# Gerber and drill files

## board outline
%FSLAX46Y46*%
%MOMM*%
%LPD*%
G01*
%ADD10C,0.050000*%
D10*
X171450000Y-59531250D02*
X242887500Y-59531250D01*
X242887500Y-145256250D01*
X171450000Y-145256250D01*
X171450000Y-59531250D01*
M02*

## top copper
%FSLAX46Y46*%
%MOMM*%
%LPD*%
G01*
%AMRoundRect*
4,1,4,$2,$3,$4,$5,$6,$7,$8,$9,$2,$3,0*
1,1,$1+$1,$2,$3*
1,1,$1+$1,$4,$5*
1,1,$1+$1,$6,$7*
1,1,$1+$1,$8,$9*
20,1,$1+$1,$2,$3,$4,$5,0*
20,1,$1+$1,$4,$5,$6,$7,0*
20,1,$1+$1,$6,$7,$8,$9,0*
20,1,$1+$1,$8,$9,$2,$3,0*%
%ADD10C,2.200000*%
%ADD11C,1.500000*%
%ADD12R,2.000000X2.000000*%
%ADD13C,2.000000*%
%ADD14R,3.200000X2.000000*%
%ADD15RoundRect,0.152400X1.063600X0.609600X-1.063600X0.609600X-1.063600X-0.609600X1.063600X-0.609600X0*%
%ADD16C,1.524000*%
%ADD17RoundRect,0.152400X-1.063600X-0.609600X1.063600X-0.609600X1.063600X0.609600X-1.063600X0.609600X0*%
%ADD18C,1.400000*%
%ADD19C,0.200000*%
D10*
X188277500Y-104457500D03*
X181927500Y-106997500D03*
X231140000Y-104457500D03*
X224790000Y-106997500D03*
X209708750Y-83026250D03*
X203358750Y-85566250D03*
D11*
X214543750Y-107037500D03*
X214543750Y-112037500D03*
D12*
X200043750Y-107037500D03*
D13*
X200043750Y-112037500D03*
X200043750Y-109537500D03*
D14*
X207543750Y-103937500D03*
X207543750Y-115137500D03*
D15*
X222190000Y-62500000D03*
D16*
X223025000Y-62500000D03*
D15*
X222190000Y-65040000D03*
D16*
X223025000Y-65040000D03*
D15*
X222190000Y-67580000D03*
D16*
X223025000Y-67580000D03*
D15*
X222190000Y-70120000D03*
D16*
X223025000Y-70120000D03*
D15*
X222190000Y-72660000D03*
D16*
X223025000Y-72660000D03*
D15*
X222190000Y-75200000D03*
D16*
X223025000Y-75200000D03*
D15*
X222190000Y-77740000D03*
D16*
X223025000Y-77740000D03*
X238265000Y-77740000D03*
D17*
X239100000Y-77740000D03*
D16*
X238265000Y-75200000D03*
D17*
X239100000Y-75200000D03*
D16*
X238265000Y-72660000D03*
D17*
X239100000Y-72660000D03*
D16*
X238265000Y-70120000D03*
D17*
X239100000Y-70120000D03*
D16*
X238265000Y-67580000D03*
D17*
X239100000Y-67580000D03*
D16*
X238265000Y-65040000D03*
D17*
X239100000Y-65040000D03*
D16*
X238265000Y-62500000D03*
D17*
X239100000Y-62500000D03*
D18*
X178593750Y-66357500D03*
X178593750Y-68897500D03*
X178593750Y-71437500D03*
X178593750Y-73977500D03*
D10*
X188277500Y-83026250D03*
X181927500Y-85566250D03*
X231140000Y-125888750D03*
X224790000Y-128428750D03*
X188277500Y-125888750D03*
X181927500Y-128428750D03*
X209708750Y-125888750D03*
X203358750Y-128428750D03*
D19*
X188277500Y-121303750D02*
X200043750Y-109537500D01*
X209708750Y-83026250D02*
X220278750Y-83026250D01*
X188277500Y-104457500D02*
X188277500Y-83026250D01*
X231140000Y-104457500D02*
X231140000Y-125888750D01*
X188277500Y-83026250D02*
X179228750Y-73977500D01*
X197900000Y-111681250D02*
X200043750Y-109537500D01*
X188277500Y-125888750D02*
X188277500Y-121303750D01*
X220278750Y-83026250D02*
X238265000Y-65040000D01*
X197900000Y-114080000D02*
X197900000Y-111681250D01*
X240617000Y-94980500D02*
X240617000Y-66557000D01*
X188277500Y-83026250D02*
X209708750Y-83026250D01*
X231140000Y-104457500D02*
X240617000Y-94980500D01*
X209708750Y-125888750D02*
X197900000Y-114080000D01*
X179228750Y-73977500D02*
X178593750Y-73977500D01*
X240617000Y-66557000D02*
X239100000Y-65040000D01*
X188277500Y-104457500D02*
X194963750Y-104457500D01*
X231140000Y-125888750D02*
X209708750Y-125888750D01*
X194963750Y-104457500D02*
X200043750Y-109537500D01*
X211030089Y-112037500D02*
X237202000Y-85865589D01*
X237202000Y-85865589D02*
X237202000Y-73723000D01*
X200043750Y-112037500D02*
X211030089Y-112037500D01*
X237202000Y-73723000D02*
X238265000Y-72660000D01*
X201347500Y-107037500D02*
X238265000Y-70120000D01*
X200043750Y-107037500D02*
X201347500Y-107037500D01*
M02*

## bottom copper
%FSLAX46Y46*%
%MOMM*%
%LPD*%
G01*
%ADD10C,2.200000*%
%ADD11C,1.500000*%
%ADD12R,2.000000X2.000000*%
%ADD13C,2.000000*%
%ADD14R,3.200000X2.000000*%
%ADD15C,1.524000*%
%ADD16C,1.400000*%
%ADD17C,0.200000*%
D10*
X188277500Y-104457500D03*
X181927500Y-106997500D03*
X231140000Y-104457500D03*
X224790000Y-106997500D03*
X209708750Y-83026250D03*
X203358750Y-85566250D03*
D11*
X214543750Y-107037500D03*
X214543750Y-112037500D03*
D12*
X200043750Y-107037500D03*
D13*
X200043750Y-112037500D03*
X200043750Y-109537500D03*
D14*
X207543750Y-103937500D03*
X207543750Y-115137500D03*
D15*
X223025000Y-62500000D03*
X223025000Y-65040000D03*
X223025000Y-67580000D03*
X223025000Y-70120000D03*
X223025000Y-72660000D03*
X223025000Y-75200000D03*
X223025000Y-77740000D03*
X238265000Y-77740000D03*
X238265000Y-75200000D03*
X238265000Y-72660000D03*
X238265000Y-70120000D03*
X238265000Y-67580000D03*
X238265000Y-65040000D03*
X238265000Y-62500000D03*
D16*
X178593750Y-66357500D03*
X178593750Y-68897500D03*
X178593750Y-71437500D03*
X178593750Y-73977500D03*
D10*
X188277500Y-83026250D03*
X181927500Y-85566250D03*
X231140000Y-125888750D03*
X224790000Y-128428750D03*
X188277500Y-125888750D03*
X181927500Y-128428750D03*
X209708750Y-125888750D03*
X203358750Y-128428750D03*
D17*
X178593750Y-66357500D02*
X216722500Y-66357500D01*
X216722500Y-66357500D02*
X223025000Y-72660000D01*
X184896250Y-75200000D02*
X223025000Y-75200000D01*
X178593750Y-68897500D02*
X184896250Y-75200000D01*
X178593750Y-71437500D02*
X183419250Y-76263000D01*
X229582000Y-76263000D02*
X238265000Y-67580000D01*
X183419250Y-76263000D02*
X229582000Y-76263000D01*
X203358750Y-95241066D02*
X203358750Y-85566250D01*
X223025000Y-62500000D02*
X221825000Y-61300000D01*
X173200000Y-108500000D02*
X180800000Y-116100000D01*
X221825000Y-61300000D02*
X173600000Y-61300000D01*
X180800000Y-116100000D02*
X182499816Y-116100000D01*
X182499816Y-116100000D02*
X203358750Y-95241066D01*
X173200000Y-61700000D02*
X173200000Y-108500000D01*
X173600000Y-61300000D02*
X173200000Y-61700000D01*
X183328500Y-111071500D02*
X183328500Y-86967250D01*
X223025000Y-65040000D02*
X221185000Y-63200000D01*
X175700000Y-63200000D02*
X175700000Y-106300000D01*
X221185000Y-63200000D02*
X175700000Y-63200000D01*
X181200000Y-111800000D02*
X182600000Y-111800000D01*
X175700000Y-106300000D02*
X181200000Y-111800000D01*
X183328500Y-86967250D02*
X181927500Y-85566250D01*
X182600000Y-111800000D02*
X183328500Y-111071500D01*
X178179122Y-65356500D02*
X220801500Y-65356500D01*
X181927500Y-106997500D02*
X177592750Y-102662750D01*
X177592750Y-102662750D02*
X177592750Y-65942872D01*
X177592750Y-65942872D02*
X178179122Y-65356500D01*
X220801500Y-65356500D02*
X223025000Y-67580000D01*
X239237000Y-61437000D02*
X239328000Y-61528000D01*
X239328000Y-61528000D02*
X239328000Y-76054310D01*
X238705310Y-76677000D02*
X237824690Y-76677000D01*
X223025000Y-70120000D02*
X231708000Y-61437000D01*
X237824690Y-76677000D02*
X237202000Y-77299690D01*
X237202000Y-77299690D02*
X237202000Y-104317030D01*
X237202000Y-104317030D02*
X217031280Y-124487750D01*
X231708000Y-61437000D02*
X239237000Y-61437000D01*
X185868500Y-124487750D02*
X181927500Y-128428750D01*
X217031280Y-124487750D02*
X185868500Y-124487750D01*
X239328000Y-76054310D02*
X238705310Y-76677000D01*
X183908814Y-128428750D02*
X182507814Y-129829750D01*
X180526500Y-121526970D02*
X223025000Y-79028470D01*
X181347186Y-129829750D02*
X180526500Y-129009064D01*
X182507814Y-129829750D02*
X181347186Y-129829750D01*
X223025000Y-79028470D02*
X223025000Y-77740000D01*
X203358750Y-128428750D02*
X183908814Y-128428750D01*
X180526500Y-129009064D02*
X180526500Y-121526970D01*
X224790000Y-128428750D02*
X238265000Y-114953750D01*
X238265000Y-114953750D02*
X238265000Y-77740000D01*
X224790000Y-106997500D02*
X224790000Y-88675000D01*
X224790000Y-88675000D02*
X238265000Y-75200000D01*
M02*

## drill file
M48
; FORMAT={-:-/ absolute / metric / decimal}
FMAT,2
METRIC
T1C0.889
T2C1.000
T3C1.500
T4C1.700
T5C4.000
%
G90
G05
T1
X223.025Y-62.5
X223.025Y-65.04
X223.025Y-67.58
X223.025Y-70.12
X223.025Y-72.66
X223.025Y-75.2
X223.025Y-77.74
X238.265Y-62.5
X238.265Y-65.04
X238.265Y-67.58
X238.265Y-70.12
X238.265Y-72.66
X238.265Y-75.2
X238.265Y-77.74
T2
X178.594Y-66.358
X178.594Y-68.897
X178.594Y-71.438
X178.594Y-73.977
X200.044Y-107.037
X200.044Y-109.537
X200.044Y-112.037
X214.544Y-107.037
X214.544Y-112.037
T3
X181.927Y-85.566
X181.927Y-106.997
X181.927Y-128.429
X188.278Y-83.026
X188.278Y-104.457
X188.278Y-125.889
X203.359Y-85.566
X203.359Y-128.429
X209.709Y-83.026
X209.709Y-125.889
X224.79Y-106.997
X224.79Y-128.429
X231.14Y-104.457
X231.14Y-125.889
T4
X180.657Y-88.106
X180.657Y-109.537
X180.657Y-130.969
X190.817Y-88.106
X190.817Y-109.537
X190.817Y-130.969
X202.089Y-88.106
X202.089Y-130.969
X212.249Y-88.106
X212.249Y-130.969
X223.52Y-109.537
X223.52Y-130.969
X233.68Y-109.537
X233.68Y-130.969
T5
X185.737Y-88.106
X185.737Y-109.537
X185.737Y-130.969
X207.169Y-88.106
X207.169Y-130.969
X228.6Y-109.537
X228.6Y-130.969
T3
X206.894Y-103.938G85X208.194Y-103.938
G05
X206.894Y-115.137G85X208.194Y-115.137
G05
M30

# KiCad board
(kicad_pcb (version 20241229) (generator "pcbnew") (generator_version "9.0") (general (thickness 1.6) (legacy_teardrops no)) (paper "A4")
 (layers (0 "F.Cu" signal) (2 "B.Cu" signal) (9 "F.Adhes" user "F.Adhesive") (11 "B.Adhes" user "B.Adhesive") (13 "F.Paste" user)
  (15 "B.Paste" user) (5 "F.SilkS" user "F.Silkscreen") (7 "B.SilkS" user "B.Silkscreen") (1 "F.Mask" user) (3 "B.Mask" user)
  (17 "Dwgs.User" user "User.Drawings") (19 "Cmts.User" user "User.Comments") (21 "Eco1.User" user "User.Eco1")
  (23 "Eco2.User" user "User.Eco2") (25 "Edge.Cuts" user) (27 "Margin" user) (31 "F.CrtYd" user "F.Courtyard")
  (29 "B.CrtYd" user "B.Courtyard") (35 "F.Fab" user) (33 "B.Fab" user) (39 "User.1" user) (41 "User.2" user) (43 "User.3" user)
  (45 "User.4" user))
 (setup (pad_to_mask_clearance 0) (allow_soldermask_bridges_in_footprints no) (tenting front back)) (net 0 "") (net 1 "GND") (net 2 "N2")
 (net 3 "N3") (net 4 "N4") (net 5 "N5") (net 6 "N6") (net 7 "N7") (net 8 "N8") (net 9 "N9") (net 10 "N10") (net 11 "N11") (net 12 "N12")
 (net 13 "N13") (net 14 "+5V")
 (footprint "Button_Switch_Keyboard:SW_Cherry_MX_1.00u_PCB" (layer "F.Cu") (at 188.2775 104.4575)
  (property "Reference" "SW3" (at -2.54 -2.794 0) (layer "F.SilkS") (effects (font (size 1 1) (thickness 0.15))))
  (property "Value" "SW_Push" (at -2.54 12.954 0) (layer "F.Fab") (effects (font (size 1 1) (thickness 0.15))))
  (pad "" np_thru_hole circle (at -7.62 5.08) (size 1.7 1.7) (drill 1.7) (layers "*.Cu" "*.Mask"))
  (pad "" np_thru_hole circle (at -2.54 5.08) (size 4 4) (drill 4) (layers "*.Cu" "*.Mask"))
  (pad "" np_thru_hole circle (at 2.54 5.08) (size 1.7 1.7) (drill 1.7) (layers "*.Cu" "*.Mask"))
  (pad "1" thru_hole circle (at 0 0) (size 2.2 2.2) (drill 1.5) (layers "*.Cu" "*.Mask") (remove_unused_layers no) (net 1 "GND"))
  (pad "2" thru_hole circle (at -6.35 2.54) (size 2.2 2.2) (drill 1.5) (layers "*.Cu" "*.Mask") (remove_unused_layers no) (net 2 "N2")))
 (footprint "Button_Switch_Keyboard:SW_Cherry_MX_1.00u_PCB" (layer "F.Cu") (at 231.14 104.4575)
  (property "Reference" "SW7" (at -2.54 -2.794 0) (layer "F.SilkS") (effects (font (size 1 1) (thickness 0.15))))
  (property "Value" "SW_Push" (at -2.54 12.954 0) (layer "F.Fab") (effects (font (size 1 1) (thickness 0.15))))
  (pad "" np_thru_hole circle (at -7.62 5.08) (size 1.7 1.7) (drill 1.7) (layers "*.Cu" "*.Mask"))
  (pad "" np_thru_hole circle (at -2.54 5.08) (size 4 4) (drill 4) (layers "*.Cu" "*.Mask"))
  (pad "" np_thru_hole circle (at 2.54 5.08) (size 1.7 1.7) (drill 1.7) (layers "*.Cu" "*.Mask"))
  (pad "1" thru_hole circle (at 0 0) (size 2.2 2.2) (drill 1.5) (layers "*.Cu" "*.Mask") (remove_unused_layers no) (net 1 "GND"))
  (pad "2" thru_hole circle (at -6.35 2.54) (size 2.2 2.2) (drill 1.5) (layers "*.Cu" "*.Mask") (remove_unused_layers no) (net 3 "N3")))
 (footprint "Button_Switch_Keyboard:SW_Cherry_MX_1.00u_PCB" (layer "F.Cu") (at 209.70875 83.02625)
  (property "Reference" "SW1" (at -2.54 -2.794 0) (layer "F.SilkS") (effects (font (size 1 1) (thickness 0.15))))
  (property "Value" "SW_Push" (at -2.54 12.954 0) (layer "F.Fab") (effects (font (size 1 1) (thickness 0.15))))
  (pad "" np_thru_hole circle (at -7.62 5.08) (size 1.7 1.7) (drill 1.7) (layers "*.Cu" "*.Mask"))
  (pad "" np_thru_hole circle (at -2.54 5.08) (size 4 4) (drill 4) (layers "*.Cu" "*.Mask"))
  (pad "" np_thru_hole circle (at 2.54 5.08) (size 1.7 1.7) (drill 1.7) (layers "*.Cu" "*.Mask"))
  (pad "1" thru_hole circle (at 0 0) (size 2.2 2.2) (drill 1.5) (layers "*.Cu" "*.Mask") (remove_unused_layers no) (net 1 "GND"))
  (pad "2" thru_hole circle (at -6.35 2.54) (size 2.2 2.2) (drill 1.5) (layers "*.Cu" "*.Mask") (remove_unused_layers no) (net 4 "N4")))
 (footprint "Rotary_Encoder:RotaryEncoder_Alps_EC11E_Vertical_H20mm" (layer "F.Cu") (at 200.04375 107.0375)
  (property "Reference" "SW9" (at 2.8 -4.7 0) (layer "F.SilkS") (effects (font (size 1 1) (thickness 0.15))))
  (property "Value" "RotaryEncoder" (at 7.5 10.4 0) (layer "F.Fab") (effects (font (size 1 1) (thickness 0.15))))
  (pad "" thru_hole circle (at 14.5 0) (size 1.5 1.5) (drill 1) (layers "*.Cu" "*.Mask") (remove_unused_layers no))
  (pad "" thru_hole circle (at 14.5 5) (size 1.5 1.5) (drill 1) (layers "*.Cu" "*.Mask") (remove_unused_layers no))
  (pad "A" thru_hole rect (at 0 0) (size 2 2) (drill 1) (layers "*.Cu" "*.Mask") (remove_unused_layers no) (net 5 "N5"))
  (pad "B" thru_hole circle (at 0 5) (size 2 2) (drill 1) (layers "*.Cu" "*.Mask") (remove_unused_layers no) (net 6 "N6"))
  (pad "C" thru_hole circle (at 0 2.5) (size 2 2) (drill 1) (layers "*.Cu" "*.Mask") (remove_unused_layers no) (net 1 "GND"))
  (pad "MP" thru_hole rect (at 7.5 -3.1) (size 3.2 2) (drill oval 2.8 1.5) (layers "*.Cu" "*.Mask") (remove_unused_layers no))
  (pad "MP" thru_hole rect (at 7.5 8.1) (size 3.2 2) (drill oval 2.8 1.5) (layers "*.Cu" "*.Mask") (remove_unused_layers no)))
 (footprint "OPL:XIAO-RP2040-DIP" (layer "F.Cu") (at 230.645 70.12)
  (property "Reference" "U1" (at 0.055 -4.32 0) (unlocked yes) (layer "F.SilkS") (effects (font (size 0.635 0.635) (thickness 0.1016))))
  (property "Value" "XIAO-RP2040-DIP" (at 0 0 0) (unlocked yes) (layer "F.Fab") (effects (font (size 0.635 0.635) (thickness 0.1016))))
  (pad "1" smd roundrect (at -8.455 -7.62 180) (size 2.432 1.524) (layers "F.Cu" "F.Mask") (roundrect_rratio 0.1) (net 4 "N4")
   (thermal_bridge_angle 45))
  (pad "1" thru_hole circle (at -7.62 -7.62 180) (size 1.524 1.524) (drill 0.889) (layers "*.Cu" "*.Mask") (remove_unused_layers no)
   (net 4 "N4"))
  (pad "2" smd roundrect (at -8.455 -5.08 180) (size 2.432 1.524) (layers "F.Cu" "F.Mask") (roundrect_rratio 0.1) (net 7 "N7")
   (thermal_bridge_angle 45))
  (pad "2" thru_hole circle (at -7.62 -5.08 180) (size 1.524 1.524) (drill 0.889) (layers "*.Cu" "*.Mask") (remove_unused_layers no)
   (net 7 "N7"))
  (pad "3" smd roundrect (at -8.455 -2.54 180) (size 2.432 1.524) (layers "F.Cu" "F.Mask") (roundrect_rratio 0.1) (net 2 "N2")
   (thermal_bridge_angle 45))
  (pad "3" thru_hole circle (at -7.62 -2.54 180) (size 1.524 1.524) (drill 0.889) (layers "*.Cu" "*.Mask") (remove_unused_layers no)
   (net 2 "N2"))
  (pad "4" smd roundrect (at -8.455 0 180) (size 2.432 1.524) (layers "F.Cu" "F.Mask") (roundrect_rratio 0.1) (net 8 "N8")
   (thermal_bridge_angle 45))
  (pad "4" thru_hole circle (at -7.62 0 180) (size 1.524 1.524) (drill 0.889) (layers "*.Cu" "*.Mask") (remove_unused_layers no)
   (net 8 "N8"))
  (pad "5" smd roundrect (at -8.455 2.54 180) (size 2.432 1.524) (layers "F.Cu" "F.Mask") (roundrect_rratio 0.1) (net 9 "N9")
   (thermal_bridge_angle 45))
  (pad "5" thru_hole circle (at -7.62 2.54 180) (size 1.524 1.524) (drill 0.889) (layers "*.Cu" "*.Mask") (remove_unused_layers no)
   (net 9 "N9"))
  (pad "6" smd roundrect (at -8.455 5.08 180) (size 2.432 1.524) (layers "F.Cu" "F.Mask") (roundrect_rratio 0.1) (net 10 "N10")
   (thermal_bridge_angle 45))
  (pad "6" thru_hole circle (at -7.62 5.08 180) (size 1.524 1.524) (drill 0.889) (layers "*.Cu" "*.Mask") (remove_unused_layers no)
   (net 10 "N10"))
  (pad "7" smd roundrect (at -8.455 7.62 180) (size 2.432 1.524) (layers "F.Cu" "F.Mask") (roundrect_rratio 0.1) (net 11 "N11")
   (thermal_bridge_angle 45))
  (pad "7" thru_hole circle (at -7.62 7.62 180) (size 1.524 1.524) (drill 0.889) (layers "*.Cu" "*.Mask") (remove_unused_layers no)
   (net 11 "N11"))
  (pad "8" thru_hole circle (at 7.62 7.62) (size 1.524 1.524) (drill 0.889) (layers "*.Cu" "*.Mask") (remove_unused_layers no)
   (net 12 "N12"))
  (pad "8" smd roundrect (at 8.455 7.62) (size 2.432 1.524) (layers "F.Cu" "F.Mask") (roundrect_rratio 0.1) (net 12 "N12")
   (thermal_bridge_angle 45))
  (pad "9" thru_hole circle (at 7.62 5.08) (size 1.524 1.524) (drill 0.889) (layers "*.Cu" "*.Mask") (remove_unused_layers no) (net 3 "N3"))
  (pad "9" smd roundrect (at 8.455 5.08) (size 2.432 1.524) (layers "F.Cu" "F.Mask") (roundrect_rratio 0.1) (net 3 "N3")
   (thermal_bridge_angle 45))
  (pad "10" thru_hole circle (at 7.62 2.54) (size 1.524 1.524) (drill 0.889) (layers "*.Cu" "*.Mask") (remove_unused_layers no) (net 6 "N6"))
  (pad "10" smd roundrect (at 8.455 2.54) (size 2.432 1.524) (layers "F.Cu" "F.Mask") (roundrect_rratio 0.1) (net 6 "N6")
   (thermal_bridge_angle 45))
  (pad "11" thru_hole circle (at 7.62 0) (size 1.524 1.524) (drill 0.889) (layers "*.Cu" "*.Mask") (remove_unused_layers no) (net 5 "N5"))
  (pad "11" smd roundrect (at 8.455 0) (size 2.432 1.524) (layers "F.Cu" "F.Mask") (roundrect_rratio 0.1) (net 5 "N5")
   (thermal_bridge_angle 45))
  (pad "12" thru_hole circle (at 7.62 -2.54) (size 1.524 1.524) (drill 0.889) (layers "*.Cu" "*.Mask") (remove_unused_layers no)
   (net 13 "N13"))
  (pad "12" smd roundrect (at 8.455 -2.54) (size 2.432 1.524) (layers "F.Cu" "F.Mask") (roundrect_rratio 0.1) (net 13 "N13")
   (thermal_bridge_angle 45))
  (pad "13" thru_hole circle (at 7.62 -5.08) (size 1.524 1.524) (drill 0.889) (layers "*.Cu" "*.Mask") (remove_unused_layers no)
   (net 1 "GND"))
  (pad "13" smd roundrect (at 8.455 -5.08) (size 2.432 1.524) (layers "F.Cu" "F.Mask") (roundrect_rratio 0.1) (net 1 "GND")
   (thermal_bridge_angle 45))
  (pad "14" thru_hole circle (at 7.62 -7.62) (size 1.524 1.524) (drill 0.889) (layers "*.Cu" "*.Mask") (remove_unused_layers no)
   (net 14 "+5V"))
  (pad "14" smd roundrect (at 8.455 -7.62) (size 2.432 1.524) (layers "F.Cu" "F.Mask") (roundrect_rratio 0.1) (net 14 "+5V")
   (thermal_bridge_angle 45)))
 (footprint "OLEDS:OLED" (layer "F.Cu") (at 178.59375 70.1675 -90)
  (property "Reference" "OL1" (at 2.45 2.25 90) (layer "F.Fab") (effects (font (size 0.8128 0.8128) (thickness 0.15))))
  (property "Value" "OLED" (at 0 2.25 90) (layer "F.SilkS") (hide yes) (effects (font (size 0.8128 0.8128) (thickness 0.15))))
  (pad "1" thru_hole circle (at -3.81 0 270) (size 1.4 1.4) (drill 1) (layers "*.Cu" "*.Mask") (remove_unused_layers no) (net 9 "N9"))
  (pad "2" thru_hole circle (at -1.27 0 270) (size 1.4 1.4) (drill 1) (layers "*.Cu" "*.Mask") (remove_unused_layers no) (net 10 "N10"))
  (pad "3" thru_hole circle (at 1.27 0 270) (size 1.4 1.4) (drill 1) (layers "*.Cu" "*.Mask") (remove_unused_layers no) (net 13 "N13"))
  (pad "4" thru_hole circle (at 3.81 0 270) (size 1.4 1.4) (drill 1) (layers "*.Cu" "*.Mask") (remove_unused_layers no) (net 1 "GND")))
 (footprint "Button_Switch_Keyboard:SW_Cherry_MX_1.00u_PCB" (layer "F.Cu") (at 188.2775 83.02625)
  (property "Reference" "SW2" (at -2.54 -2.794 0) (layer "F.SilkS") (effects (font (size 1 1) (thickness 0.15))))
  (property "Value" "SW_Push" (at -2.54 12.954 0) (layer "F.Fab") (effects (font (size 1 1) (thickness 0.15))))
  (pad "" np_thru_hole circle (at -7.62 5.08) (size 1.7 1.7) (drill 1.7) (layers "*.Cu" "*.Mask"))
  (pad "" np_thru_hole circle (at -2.54 5.08) (size 4 4) (drill 4) (layers "*.Cu" "*.Mask"))
  (pad "" np_thru_hole circle (at 2.54 5.08) (size 1.7 1.7) (drill 1.7) (layers "*.Cu" "*.Mask"))
  (pad "1" thru_hole circle (at 0 0) (size 2.2 2.2) (drill 1.5) (layers "*.Cu" "*.Mask") (remove_unused_layers no) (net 1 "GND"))
  (pad "2" thru_hole circle (at -6.35 2.54) (size 2.2 2.2) (drill 1.5) (layers "*.Cu" "*.Mask") (remove_unused_layers no) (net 7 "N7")))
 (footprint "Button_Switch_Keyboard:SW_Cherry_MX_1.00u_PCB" (layer "F.Cu") (at 231.14 125.88875)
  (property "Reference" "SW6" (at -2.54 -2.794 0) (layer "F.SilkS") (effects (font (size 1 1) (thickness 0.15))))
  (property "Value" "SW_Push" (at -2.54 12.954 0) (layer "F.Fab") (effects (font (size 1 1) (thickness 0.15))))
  (pad "" np_thru_hole circle (at -7.62 5.08) (size 1.7 1.7) (drill 1.7) (layers "*.Cu" "*.Mask"))
  (pad "" np_thru_hole circle (at -2.54 5.08) (size 4 4) (drill 4) (layers "*.Cu" "*.Mask"))
  (pad "" np_thru_hole circle (at 2.54 5.08) (size 1.7 1.7) (drill 1.7) (layers "*.Cu" "*.Mask"))
  (pad "1" thru_hole circle (at 0 0) (size 2.2 2.2) (drill 1.5) (layers "*.Cu" "*.Mask") (remove_unused_layers no) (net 1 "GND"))
  (pad "2" thru_hole circle (at -6.35 2.54) (size 2.2 2.2) (drill 1.5) (layers "*.Cu" "*.Mask") (remove_unused_layers no) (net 12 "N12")))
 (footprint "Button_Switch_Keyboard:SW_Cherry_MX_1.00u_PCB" (layer "F.Cu") (at 188.2775 125.88875)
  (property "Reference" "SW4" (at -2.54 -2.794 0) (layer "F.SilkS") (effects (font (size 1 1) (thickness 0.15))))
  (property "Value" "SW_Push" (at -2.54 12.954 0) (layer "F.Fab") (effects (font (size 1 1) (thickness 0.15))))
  (pad "" np_thru_hole circle (at -7.62 5.08) (size 1.7 1.7) (drill 1.7) (layers "*.Cu" "*.Mask"))
  (pad "" np_thru_hole circle (at -2.54 5.08) (size 4 4) (drill 4) (layers "*.Cu" "*.Mask"))
  (pad "" np_thru_hole circle (at 2.54 5.08) (size 1.7 1.7) (drill 1.7) (layers "*.Cu" "*.Mask"))
  (pad "1" thru_hole circle (at 0 0) (size 2.2 2.2) (drill 1.5) (layers "*.Cu" "*.Mask") (remove_unused_layers no) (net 1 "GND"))
  (pad "2" thru_hole circle (at -6.35 2.54) (size 2.2 2.2) (drill 1.5) (layers "*.Cu" "*.Mask") (remove_unused_layers no) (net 8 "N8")))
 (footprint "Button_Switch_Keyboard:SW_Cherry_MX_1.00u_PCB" (layer "F.Cu") (at 209.70875 125.88875)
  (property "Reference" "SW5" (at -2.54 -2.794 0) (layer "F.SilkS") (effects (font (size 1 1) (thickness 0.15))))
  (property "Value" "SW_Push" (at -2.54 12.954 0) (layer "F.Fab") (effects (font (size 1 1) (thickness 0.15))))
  (pad "" np_thru_hole circle (at -7.62 5.08) (size 1.7 1.7) (drill 1.7) (layers "*.Cu" "*.Mask"))
  (pad "" np_thru_hole circle (at -2.54 5.08) (size 4 4) (drill 4) (layers "*.Cu" "*.Mask"))
  (pad "" np_thru_hole circle (at 2.54 5.08) (size 1.7 1.7) (drill 1.7) (layers "*.Cu" "*.Mask"))
  (pad "1" thru_hole circle (at 0 0) (size 2.2 2.2) (drill 1.5) (layers "*.Cu" "*.Mask") (remove_unused_layers no) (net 1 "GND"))
  (pad "2" thru_hole circle (at -6.35 2.54) (size 2.2 2.2) (drill 1.5) (layers "*.Cu" "*.Mask") (remove_unused_layers no) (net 11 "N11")))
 (gr_rect (start 171.45 59.53125) (end 242.8875 145.25625) (stroke (width 0.05) (type default)) (fill no) (layer "Edge.Cuts"))
 (segment (start 178.59375 66.3575) (end 216.7225 66.3575) (width 0.2) (layer "B.Cu") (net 9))
 (segment (start 216.7225 66.3575) (end 223.025 72.66) (width 0.2) (layer "B.Cu") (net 9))
 (segment (start 184.89625 75.2) (end 223.025 75.2) (width 0.2) (layer "B.Cu") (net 10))
 (segment (start 178.59375 68.8975) (end 184.89625 75.2) (width 0.2) (layer "B.Cu") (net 10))
 (segment (start 178.59375 71.4375) (end 183.41925 76.263) (width 0.2) (layer "B.Cu") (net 13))
 (segment (start 229.582 76.263) (end 238.265 67.58) (width 0.2) (layer "B.Cu") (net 13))
 (segment (start 183.41925 76.263) (end 229.582 76.263) (width 0.2) (layer "B.Cu") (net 13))
 (segment (start 188.2775 121.30375) (end 200.04375 109.5375) (width 0.2) (layer "F.Cu") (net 1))
 (segment (start 209.70875 83.02625) (end 220.27875 83.02625) (width 0.2) (layer "F.Cu") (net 1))
 (segment (start 188.2775 104.4575) (end 188.2775 83.02625) (width 0.2) (layer "F.Cu") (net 1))
 (segment (start 231.14 104.4575) (end 231.14 125.88875) (width 0.2) (layer "F.Cu") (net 1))
 (segment (start 188.2775 83.02625) (end 179.22875 73.9775) (width 0.2) (layer "F.Cu") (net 1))
 (segment (start 197.9 111.68125) (end 200.04375 109.5375) (width 0.2) (layer "F.Cu") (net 1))
 (segment (start 188.2775 125.88875) (end 188.2775 121.30375) (width 0.2) (layer "F.Cu") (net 1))
 (segment (start 220.27875 83.02625) (end 238.265 65.04) (width 0.2) (layer "F.Cu") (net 1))
 (segment (start 197.9 114.08) (end 197.9 111.68125) (width 0.2) (layer "F.Cu") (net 1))
 (segment (start 240.617 94.9805) (end 240.617 66.557) (width 0.2) (layer "F.Cu") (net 1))
 (segment (start 188.2775 83.02625) (end 209.70875 83.02625) (width 0.2) (layer "F.Cu") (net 1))
 (segment (start 231.14 104.4575) (end 240.617 94.9805) (width 0.2) (layer "F.Cu") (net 1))
 (segment (start 209.70875 125.88875) (end 197.9 114.08) (width 0.2) (layer "F.Cu") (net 1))
 (segment (start 179.22875 73.9775) (end 178.59375 73.9775) (width 0.2) (layer "F.Cu") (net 1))
 (segment (start 240.617 66.557) (end 239.1 65.04) (width 0.2) (layer "F.Cu") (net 1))
 (segment (start 188.2775 104.4575) (end 194.96375 104.4575) (width 0.2) (layer "F.Cu") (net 1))
 (segment (start 231.14 125.88875) (end 209.70875 125.88875) (width 0.2) (layer "F.Cu") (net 1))
 (segment (start 194.96375 104.4575) (end 200.04375 109.5375) (width 0.2) (layer "F.Cu") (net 1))
 (segment (start 203.35875 95.241066) (end 203.35875 85.56625) (width 0.2) (layer "B.Cu") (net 4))
 (segment (start 223.025 62.5) (end 221.825 61.3) (width 0.2) (layer "B.Cu") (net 4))
 (segment (start 173.2 108.5) (end 180.8 116.1) (width 0.2) (layer "B.Cu") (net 4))
 (segment (start 221.825 61.3) (end 173.6 61.3) (width 0.2) (layer "B.Cu") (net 4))
 (segment (start 180.8 116.1) (end 182.499816 116.1) (width 0.2) (layer "B.Cu") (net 4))
 (segment (start 182.499816 116.1) (end 203.35875 95.241066) (width 0.2) (layer "B.Cu") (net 4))
 (segment (start 173.2 61.7) (end 173.2 108.5) (width 0.2) (layer "B.Cu") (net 4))
 (segment (start 173.6 61.3) (end 173.2 61.7) (width 0.2) (layer "B.Cu") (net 4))
 (segment (start 183.3285 111.0715) (end 183.3285 86.96725) (width 0.2) (layer "B.Cu") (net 7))
 (segment (start 223.025 65.04) (end 221.185 63.2) (width 0.2) (layer "B.Cu") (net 7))
 (segment (start 175.7 63.2) (end 175.7 106.3) (width 0.2) (layer "B.Cu") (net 7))
 (segment (start 221.185 63.2) (end 175.7 63.2) (width 0.2) (layer "B.Cu") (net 7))
 (segment (start 181.2 111.8) (end 182.6 111.8) (width 0.2) (layer "B.Cu") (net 7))
 (segment (start 175.7 106.3) (end 181.2 111.8) (width 0.2) (layer "B.Cu") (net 7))
 (segment (start 183.3285 86.96725) (end 181.9275 85.56625) (width 0.2) (layer "B.Cu") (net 7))
 (segment (start 182.6 111.8) (end 183.3285 111.0715) (width 0.2) (layer "B.Cu") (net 7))
 (segment (start 178.179122 65.3565) (end 220.8015 65.3565) (width 0.2) (layer "B.Cu") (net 2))
 (segment (start 181.9275 106.9975) (end 177.59275 102.66275) (width 0.2) (layer "B.Cu") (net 2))
 (segment (start 177.59275 102.66275) (end 177.59275 65.942872) (width 0.2) (layer "B.Cu") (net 2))
 (segment (start 177.59275 65.942872) (end 178.179122 65.3565) (width 0.2) (layer "B.Cu") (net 2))
 (segment (start 220.8015 65.3565) (end 223.025 67.58) (width 0.2) (layer "B.Cu") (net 2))
 (segment (start 239.237 61.437) (end 239.328 61.528) (width 0.2) (layer "B.Cu") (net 8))
 (segment (start 239.328 61.528) (end 239.328 76.05431) (width 0.2) (layer "B.Cu") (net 8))
 (segment (start 238.70531 76.677) (end 237.82469 76.677) (width 0.2) (layer "B.Cu") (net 8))
 (segment (start 223.025 70.12) (end 231.708 61.437) (width 0.2) (layer "B.Cu") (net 8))
 (segment (start 237.82469 76.677) (end 237.202 77.29969) (width 0.2) (layer "B.Cu") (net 8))
 (segment (start 237.202 77.29969) (end 237.202 104.31703) (width 0.2) (layer "B.Cu") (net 8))
 (segment (start 237.202 104.31703) (end 217.03128 124.48775) (width 0.2) (layer "B.Cu") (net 8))
 (segment (start 231.708 61.437) (end 239.237 61.437) (width 0.2) (layer "B.Cu") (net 8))
 (segment (start 185.8685 124.48775) (end 181.9275 128.42875) (width 0.2) (layer "B.Cu") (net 8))
 (segment (start 217.03128 124.48775) (end 185.8685 124.48775) (width 0.2) (layer "B.Cu") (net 8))
 (segment (start 239.328 76.05431) (end 238.70531 76.677) (width 0.2) (layer "B.Cu") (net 8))
 (segment (start 183.908814 128.42875) (end 182.507814 129.82975) (width 0.2) (layer "B.Cu") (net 11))
 (segment (start 180.5265 121.52697) (end 223.025 79.02847) (width 0.2) (layer "B.Cu") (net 11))
 (segment (start 181.347186 129.82975) (end 180.5265 129.009064) (width 0.2) (layer "B.Cu") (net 11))
 (segment (start 182.507814 129.82975) (end 181.347186 129.82975) (width 0.2) (layer "B.Cu") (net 11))
 (segment (start 223.025 79.02847) (end 223.025 77.74) (width 0.2) (layer "B.Cu") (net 11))
 (segment (start 203.35875 128.42875) (end 183.908814 128.42875) (width 0.2) (layer "B.Cu") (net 11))
 (segment (start 180.5265 129.009064) (end 180.5265 121.52697) (width 0.2) (layer "B.Cu") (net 11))
 (segment (start 224.79 128.42875) (end 238.265 114.95375) (width 0.2) (layer "B.Cu") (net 12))
 (segment (start 238.265 114.95375) (end 238.265 77.74) (width 0.2) (layer "B.Cu") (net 12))
 (segment (start 224.79 106.9975) (end 224.79 88.675) (width 0.2) (layer "B.Cu") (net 3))
 (segment (start 224.79 88.675) (end 238.265 75.2) (width 0.2) (layer "B.Cu") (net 3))
 (segment (start 211.030089 112.0375) (end 237.202 85.865589) (width 0.2) (layer "F.Cu") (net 6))
 (segment (start 237.202 85.865589) (end 237.202 73.723) (width 0.2) (layer "F.Cu") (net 6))
 (segment (start 200.04375 112.0375) (end 211.030089 112.0375) (width 0.2) (layer "F.Cu") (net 6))
 (segment (start 237.202 73.723) (end 238.265 72.66) (width 0.2) (layer "F.Cu") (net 6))
 (segment (start 201.3475 107.0375) (end 238.265 70.12) (width 0.2) (layer "F.Cu") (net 5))
 (segment (start 200.04375 107.0375) (end 201.3475 107.0375) (width 0.2) (layer "F.Cu") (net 5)))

